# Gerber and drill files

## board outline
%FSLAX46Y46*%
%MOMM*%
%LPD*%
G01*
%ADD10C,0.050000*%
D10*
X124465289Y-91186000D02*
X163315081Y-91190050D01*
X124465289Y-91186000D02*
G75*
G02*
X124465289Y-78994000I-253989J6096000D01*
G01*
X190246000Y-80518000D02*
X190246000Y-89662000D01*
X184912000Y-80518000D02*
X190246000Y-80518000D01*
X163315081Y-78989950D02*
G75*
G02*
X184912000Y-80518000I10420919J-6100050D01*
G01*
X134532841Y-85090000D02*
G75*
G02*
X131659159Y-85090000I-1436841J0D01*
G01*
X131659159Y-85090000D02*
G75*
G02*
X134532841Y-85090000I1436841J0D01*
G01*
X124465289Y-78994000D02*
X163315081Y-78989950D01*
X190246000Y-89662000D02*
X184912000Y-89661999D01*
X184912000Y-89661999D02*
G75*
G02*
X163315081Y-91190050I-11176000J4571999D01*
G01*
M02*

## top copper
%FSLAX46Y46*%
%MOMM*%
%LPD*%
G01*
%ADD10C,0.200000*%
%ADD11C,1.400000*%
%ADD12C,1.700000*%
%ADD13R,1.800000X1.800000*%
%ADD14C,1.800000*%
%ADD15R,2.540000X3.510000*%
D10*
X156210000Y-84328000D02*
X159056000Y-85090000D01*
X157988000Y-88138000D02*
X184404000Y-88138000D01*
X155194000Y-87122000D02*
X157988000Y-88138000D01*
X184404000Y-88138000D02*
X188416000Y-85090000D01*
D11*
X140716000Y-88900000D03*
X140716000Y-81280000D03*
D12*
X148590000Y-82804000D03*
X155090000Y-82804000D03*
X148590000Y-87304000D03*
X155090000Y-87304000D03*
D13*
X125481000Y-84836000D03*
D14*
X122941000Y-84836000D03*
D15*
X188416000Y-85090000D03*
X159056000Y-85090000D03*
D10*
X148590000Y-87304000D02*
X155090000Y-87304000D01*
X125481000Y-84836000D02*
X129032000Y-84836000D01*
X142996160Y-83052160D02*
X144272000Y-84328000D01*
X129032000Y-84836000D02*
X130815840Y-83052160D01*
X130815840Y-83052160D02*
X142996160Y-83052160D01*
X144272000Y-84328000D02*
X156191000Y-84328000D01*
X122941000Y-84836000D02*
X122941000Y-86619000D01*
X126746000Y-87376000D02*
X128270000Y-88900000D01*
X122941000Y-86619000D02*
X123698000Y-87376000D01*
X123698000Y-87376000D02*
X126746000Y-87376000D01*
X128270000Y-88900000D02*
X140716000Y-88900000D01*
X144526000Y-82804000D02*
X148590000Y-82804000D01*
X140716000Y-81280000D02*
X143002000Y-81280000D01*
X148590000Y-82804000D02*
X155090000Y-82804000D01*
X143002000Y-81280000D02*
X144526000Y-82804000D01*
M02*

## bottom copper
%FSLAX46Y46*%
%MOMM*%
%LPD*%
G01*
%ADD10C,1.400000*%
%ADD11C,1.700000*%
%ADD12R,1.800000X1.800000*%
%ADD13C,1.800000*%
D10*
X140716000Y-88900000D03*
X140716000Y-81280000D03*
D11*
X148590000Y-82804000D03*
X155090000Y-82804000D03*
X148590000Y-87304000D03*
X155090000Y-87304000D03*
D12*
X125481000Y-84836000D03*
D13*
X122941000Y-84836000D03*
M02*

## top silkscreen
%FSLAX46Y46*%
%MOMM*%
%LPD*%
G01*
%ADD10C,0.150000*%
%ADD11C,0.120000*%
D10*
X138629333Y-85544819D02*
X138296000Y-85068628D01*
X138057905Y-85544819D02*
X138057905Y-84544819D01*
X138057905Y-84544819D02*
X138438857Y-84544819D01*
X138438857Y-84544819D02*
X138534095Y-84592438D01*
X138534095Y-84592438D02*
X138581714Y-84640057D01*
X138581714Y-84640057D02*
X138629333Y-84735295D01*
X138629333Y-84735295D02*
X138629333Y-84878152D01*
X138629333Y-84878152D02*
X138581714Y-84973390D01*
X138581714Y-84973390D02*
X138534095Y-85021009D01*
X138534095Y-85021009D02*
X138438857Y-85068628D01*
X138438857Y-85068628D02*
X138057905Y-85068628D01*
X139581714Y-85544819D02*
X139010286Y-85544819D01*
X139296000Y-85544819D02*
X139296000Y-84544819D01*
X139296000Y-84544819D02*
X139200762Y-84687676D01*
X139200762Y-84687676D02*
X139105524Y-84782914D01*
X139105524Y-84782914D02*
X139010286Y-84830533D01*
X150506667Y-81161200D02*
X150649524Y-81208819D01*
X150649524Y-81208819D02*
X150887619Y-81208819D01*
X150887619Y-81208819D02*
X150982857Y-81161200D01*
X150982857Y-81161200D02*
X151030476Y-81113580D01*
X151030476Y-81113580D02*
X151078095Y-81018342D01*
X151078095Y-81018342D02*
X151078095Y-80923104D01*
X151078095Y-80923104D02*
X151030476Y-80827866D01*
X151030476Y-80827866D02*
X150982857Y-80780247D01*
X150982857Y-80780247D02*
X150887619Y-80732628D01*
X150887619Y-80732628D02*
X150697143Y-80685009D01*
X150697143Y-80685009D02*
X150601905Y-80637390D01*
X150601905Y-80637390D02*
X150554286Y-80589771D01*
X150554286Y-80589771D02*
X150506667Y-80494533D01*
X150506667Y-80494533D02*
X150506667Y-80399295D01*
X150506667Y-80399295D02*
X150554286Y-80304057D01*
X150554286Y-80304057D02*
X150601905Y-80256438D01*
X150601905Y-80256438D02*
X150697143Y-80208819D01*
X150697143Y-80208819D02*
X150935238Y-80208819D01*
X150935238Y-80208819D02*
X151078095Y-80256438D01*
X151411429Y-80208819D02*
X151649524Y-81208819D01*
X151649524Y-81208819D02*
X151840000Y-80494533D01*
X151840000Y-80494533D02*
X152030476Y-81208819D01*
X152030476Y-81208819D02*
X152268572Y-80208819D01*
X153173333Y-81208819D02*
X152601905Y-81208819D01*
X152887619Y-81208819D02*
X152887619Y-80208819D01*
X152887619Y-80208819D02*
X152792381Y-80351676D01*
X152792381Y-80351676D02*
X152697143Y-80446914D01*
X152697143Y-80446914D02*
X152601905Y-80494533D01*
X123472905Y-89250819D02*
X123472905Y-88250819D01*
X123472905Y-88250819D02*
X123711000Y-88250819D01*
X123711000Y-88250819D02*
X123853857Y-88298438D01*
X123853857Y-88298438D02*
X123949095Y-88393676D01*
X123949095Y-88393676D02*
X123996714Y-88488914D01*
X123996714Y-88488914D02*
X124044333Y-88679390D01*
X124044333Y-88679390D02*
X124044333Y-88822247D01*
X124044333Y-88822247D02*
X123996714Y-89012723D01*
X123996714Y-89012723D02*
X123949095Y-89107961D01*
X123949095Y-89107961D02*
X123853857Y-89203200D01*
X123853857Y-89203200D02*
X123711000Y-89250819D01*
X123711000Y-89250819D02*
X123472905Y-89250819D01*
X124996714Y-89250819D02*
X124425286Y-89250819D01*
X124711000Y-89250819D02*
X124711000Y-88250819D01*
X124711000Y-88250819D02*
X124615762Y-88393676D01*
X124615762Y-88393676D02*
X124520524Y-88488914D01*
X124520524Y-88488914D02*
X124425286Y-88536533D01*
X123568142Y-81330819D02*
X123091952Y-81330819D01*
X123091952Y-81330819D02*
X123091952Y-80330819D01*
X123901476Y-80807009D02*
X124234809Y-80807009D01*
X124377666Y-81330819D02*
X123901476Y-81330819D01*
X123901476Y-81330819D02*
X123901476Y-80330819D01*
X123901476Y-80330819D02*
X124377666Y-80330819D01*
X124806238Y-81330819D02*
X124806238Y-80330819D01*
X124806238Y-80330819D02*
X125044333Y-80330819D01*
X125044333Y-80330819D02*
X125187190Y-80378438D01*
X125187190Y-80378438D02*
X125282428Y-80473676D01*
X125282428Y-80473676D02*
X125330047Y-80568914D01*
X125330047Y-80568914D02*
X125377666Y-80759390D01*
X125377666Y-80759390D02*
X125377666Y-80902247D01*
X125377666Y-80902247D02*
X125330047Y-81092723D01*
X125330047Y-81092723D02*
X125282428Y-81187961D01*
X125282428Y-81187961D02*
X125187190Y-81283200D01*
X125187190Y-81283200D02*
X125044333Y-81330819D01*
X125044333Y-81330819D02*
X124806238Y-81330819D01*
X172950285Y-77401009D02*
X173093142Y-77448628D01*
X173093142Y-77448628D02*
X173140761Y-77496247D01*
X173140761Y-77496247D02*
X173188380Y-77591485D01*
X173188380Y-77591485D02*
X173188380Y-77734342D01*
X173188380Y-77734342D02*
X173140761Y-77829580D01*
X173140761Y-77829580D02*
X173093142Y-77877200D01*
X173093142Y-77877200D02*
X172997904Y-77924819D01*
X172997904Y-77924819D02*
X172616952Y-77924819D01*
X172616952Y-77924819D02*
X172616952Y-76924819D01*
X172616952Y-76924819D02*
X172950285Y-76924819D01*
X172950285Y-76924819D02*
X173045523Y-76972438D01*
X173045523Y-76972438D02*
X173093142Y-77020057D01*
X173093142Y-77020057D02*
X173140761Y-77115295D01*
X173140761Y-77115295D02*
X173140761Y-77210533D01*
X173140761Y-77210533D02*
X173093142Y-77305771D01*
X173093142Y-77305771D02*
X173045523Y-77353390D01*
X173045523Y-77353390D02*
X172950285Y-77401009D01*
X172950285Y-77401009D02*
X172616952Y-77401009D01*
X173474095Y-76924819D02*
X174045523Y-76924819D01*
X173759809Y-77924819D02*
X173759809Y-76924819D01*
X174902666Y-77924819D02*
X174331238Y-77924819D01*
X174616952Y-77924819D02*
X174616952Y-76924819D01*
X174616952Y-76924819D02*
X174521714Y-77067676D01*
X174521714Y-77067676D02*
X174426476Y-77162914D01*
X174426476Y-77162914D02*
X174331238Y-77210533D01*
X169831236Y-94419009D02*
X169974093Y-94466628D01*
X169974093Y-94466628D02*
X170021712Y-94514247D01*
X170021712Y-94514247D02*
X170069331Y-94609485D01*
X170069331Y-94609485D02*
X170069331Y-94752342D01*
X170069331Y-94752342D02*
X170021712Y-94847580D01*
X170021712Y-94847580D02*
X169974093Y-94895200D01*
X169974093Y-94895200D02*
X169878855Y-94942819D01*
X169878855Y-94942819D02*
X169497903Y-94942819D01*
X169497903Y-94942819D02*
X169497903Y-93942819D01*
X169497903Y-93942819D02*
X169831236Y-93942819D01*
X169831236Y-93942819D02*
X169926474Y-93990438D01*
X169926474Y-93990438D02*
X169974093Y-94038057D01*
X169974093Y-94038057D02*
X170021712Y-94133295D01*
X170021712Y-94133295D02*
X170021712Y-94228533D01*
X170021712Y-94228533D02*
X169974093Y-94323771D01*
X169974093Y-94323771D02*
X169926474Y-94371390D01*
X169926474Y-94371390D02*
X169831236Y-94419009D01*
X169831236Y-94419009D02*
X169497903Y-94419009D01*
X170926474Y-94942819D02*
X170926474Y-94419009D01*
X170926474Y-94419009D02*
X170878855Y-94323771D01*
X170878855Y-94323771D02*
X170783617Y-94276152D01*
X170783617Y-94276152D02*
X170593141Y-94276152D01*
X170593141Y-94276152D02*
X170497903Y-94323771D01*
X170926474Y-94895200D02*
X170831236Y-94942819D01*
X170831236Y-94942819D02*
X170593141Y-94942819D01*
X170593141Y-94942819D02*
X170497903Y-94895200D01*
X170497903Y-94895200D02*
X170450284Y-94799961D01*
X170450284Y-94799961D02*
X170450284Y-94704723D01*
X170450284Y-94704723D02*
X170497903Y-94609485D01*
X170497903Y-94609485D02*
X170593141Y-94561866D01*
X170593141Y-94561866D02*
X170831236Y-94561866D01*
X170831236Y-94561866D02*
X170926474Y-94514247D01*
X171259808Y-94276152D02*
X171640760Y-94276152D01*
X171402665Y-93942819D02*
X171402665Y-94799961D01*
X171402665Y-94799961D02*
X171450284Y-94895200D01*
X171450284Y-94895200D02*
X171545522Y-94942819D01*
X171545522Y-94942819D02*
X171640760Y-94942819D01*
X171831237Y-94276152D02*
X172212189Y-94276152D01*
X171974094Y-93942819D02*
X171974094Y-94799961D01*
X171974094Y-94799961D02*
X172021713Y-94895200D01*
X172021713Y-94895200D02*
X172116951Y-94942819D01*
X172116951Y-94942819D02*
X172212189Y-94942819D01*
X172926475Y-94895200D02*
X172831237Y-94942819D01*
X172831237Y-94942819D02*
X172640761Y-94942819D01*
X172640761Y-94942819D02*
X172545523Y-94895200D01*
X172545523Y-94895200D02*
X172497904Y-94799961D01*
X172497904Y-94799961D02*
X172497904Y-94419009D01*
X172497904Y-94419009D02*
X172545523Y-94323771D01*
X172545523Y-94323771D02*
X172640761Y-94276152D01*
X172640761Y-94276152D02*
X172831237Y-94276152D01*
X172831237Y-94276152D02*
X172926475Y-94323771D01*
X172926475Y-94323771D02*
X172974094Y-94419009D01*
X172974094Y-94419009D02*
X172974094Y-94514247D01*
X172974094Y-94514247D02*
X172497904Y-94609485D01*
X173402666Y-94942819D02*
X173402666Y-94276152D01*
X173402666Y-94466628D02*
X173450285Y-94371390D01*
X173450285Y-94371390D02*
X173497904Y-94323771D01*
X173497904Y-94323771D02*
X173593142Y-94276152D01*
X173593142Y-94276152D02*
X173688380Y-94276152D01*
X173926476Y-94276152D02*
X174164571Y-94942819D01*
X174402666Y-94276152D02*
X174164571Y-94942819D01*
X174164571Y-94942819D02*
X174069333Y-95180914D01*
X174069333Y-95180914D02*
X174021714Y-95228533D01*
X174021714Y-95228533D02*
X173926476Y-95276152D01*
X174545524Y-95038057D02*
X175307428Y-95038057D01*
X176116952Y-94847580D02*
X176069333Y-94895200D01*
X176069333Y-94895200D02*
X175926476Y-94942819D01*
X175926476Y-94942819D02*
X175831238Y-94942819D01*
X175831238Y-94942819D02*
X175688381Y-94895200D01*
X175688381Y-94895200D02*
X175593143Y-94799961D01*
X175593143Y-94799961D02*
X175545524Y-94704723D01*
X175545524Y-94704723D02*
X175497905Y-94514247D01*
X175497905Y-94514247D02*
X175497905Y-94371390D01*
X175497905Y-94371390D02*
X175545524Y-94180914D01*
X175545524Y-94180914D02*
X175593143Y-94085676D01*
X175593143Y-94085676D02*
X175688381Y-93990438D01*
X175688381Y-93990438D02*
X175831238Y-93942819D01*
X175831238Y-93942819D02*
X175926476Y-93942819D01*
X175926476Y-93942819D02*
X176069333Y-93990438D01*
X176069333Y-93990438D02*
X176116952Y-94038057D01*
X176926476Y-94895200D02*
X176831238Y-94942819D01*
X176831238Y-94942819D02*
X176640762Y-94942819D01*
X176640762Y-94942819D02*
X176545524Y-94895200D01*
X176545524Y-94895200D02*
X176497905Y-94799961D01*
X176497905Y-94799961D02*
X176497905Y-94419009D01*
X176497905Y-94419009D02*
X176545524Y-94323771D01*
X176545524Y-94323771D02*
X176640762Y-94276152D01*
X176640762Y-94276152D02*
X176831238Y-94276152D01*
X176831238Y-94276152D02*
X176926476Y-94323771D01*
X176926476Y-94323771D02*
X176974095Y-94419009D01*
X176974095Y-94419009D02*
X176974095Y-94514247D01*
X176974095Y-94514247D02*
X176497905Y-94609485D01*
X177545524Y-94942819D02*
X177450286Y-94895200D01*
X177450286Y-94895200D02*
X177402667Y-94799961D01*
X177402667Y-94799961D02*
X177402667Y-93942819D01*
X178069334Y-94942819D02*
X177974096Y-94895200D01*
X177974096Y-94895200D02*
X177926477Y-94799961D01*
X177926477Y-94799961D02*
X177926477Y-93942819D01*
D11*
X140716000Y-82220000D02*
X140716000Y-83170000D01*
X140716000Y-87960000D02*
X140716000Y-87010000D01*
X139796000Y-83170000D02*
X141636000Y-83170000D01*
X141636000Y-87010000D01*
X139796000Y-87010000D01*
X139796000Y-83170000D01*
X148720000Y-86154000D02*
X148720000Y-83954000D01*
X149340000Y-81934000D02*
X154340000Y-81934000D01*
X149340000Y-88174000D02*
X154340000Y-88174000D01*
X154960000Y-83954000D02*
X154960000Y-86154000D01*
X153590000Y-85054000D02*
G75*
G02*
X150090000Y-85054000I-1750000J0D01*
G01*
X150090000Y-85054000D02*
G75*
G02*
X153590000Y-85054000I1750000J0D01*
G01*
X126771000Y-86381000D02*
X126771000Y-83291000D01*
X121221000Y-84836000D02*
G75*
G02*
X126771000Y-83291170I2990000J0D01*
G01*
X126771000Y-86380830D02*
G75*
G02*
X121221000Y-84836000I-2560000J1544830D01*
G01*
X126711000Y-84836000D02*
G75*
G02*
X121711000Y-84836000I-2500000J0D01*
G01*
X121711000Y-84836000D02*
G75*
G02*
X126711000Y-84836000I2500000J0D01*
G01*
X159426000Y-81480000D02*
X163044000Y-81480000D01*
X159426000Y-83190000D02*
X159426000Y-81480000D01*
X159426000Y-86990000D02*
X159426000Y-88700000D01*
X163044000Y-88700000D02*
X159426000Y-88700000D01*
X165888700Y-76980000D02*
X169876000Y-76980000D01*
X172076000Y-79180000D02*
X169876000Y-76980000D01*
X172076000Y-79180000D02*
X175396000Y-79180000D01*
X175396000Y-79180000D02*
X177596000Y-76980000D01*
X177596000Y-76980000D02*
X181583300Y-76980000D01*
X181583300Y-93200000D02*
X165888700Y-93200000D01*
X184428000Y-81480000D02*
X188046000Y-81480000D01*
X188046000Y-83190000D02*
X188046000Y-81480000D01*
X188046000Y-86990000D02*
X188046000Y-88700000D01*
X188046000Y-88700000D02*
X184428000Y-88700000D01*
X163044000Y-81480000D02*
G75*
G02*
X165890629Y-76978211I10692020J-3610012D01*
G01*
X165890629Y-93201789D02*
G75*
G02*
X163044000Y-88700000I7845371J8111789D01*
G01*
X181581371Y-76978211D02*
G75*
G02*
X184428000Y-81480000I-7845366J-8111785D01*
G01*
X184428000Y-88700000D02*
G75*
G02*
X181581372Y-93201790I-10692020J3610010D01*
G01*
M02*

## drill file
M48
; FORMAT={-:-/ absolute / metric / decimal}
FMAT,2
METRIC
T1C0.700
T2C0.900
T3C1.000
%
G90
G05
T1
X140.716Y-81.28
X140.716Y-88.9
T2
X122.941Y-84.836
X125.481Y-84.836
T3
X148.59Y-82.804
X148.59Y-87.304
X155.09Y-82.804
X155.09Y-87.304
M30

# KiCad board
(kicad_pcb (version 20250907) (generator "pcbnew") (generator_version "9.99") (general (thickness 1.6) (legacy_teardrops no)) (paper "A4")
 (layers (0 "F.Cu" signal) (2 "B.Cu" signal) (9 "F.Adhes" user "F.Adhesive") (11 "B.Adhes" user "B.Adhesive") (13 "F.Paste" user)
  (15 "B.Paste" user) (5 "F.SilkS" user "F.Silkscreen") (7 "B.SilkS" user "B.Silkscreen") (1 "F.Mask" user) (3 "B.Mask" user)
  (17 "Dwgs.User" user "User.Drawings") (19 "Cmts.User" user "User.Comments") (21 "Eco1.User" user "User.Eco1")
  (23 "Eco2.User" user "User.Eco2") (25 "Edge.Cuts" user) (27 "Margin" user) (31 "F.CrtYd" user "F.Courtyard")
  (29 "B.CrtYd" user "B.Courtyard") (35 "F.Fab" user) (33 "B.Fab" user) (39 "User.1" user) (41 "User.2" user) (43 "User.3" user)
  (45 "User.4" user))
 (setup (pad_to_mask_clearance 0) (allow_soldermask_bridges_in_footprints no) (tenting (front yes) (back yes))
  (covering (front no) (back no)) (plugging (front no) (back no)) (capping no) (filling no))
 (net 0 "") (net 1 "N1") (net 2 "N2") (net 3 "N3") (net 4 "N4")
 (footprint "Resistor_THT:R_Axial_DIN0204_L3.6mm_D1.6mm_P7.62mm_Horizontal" (layer "F.Cu") (at 140.716 88.9 90)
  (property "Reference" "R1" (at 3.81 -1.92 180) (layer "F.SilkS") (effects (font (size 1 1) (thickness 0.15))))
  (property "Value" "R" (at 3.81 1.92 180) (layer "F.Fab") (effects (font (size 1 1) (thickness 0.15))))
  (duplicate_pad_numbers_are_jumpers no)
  (fp_line (start 6.68 0) (end 5.73 0) (stroke (width 0.12) (type solid)) (layer "F.SilkS"))
  (fp_line (start 0.94 0) (end 1.89 0) (stroke (width 0.12) (type solid)) (layer "F.SilkS"))
  (fp_rect (start 1.89 -0.92) (end 5.73 0.92) (stroke (width 0.12) (type solid)) (fill no) (layer "F.SilkS"))
  (pad "1" thru_hole circle (at 0 0 90) (size 1.4 1.4) (drill 0.7) (layers "*.Cu" "*.Mask") (remove_unused_layers no) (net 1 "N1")
   (tenting (front none) (back none)))
  (pad "2" thru_hole circle (at 7.62 0 90) (size 1.4 1.4) (drill 0.7) (layers "*.Cu" "*.Mask") (remove_unused_layers no) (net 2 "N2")
   (tenting (front none) (back none))))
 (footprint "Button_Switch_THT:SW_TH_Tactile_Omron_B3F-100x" (layer "F.Cu") (at 148.59 82.804)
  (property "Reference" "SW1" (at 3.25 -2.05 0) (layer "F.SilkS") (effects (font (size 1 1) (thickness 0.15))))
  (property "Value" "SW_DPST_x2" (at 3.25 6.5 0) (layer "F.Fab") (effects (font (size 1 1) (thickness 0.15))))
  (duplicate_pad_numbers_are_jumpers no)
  (fp_line (start 0.13 3.35) (end 0.13 1.15) (stroke (width 0.12) (type solid)) (layer "F.SilkS"))
  (fp_line (start 0.75 -0.87) (end 5.75 -0.87) (stroke (width 0.12) (type solid)) (layer "F.SilkS"))
  (fp_line (start 0.75 5.37) (end 5.75 5.37) (stroke (width 0.12) (type solid)) (layer "F.SilkS"))
  (fp_line (start 6.37 1.15) (end 6.37 3.35) (stroke (width 0.12) (type solid)) (layer "F.SilkS"))
  (fp_circle (center 3.25 2.25) (end 5 2.25) (stroke (width 0.12) (type solid)) (fill no) (layer "F.SilkS"))
  (pad "1" thru_hole circle (at 0 0) (size 1.7 1.7) (drill 1) (layers "*.Cu" "*.Mask") (remove_unused_layers no) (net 2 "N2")
   (thermal_bridge_angle 90) (tenting (front none) (back none)))
  (pad "1" thru_hole circle (at 6.5 0) (size 1.7 1.7) (drill 1) (layers "*.Cu" "*.Mask") (remove_unused_layers no) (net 2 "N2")
   (tenting (front none) (back none)))
  (pad "2" thru_hole circle (at 0 4.5) (size 1.7 1.7) (drill 1) (layers "*.Cu" "*.Mask") (remove_unused_layers no) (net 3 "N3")
   (tenting (front none) (back none)))
  (pad "2" thru_hole circle (at 6.5 4.5) (size 1.7 1.7) (drill 1) (layers "*.Cu" "*.Mask") (remove_unused_layers no) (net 3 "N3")
   (tenting (front none) (back none))))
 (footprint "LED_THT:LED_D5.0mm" (layer "F.Cu") (at 125.481 84.836 180)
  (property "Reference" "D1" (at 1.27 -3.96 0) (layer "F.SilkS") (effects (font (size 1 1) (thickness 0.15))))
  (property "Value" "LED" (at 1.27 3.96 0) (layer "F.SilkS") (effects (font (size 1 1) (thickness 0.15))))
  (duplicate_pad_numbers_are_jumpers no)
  (fp_line (start -1.29 -1.545) (end -1.29 1.545) (stroke (width 0.12) (type solid)) (layer "F.SilkS"))
  (fp_arc (start 4.26 0) (mid 2.071779 2.880495) (end -1.29 1.54483) (stroke (width 0.12) (type solid)) (layer "F.SilkS"))
  (fp_arc (start -1.29 -1.54483) (mid 2.071779 -2.880495) (end 4.26 0) (stroke (width 0.12) (type solid)) (layer "F.SilkS"))
  (fp_circle (center 1.27 0) (end 3.77 0) (stroke (width 0.12) (type solid)) (fill no) (layer "F.SilkS"))
  (pad "1" thru_hole rect (at 0 0 180) (size 1.8 1.8) (drill 0.9) (layers "*.Cu" "*.Mask") (remove_unused_layers no) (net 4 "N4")
   (tenting (front none) (back none)))
  (pad "2" thru_hole circle (at 2.54 0 180) (size 1.8 1.8) (drill 0.9) (layers "*.Cu" "*.Mask") (remove_unused_layers no) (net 1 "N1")
   (tenting (front none) (back none))))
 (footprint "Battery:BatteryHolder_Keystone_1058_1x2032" (layer "F.Cu") (at 173.736 85.09 180)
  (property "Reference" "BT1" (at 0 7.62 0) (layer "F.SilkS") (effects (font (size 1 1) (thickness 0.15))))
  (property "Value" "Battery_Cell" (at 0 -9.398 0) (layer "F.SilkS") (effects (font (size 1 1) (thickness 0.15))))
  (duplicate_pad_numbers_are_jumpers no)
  (fp_line (start 14.31 3.61) (end 10.692 3.61) (stroke (width 0.12) (type solid)) (layer "F.SilkS"))
  (fp_line (start 14.31 1.9) (end 14.31 3.61) (stroke (width 0.12) (type solid)) (layer "F.SilkS"))
  (fp_line (start 14.31 -1.9) (end 14.31 -3.61) (stroke (width 0.12) (type solid)) (layer "F.SilkS"))
  (fp_line (start 10.692 -3.61) (end 14.31 -3.61) (stroke (width 0.12) (type solid)) (layer "F.SilkS"))
  (fp_line (start 7.8473 8.11) (end 3.86 8.11) (stroke (width 0.12) (type solid)) (layer "F.SilkS"))
  (fp_line (start 1.66 5.91) (end 3.86 8.11) (stroke (width 0.12) (type solid)) (layer "F.SilkS"))
  (fp_line (start 1.66 5.91) (end -1.66 5.91) (stroke (width 0.12) (type solid)) (layer "F.SilkS"))
  (fp_line (start -1.66 5.91) (end -3.86 8.11) (stroke (width 0.12) (type solid)) (layer "F.SilkS"))
  (fp_line (start -3.86 8.11) (end -7.8473 8.11) (stroke (width 0.12) (type solid)) (layer "F.SilkS"))
  (fp_line (start -7.8473 -8.11) (end 7.8473 -8.11) (stroke (width 0.12) (type solid)) (layer "F.SilkS"))
  (fp_line (start -10.692 3.61) (end -14.31 3.61) (stroke (width 0.12) (type solid)) (layer "F.SilkS"))
  (fp_line (start -14.31 1.9) (end -14.31 3.61) (stroke (width 0.12) (type solid)) (layer "F.SilkS"))
  (fp_line (start -14.31 -1.9) (end -14.31 -3.61) (stroke (width 0.12) (type solid)) (layer "F.SilkS"))
  (fp_line (start -14.31 -3.61) (end -10.692 -3.61) (stroke (width 0.12) (type solid)) (layer "F.SilkS"))
  (fp_arc (start 10.692 3.61) (mid 9.538084 6.031244) (end 7.845371 8.111789) (stroke (width 0.12) (type solid)) (layer "F.SilkS"))
  (fp_arc (start 7.845371 -8.111789) (mid 9.538085 -6.031244) (end 10.692 -3.61) (stroke (width 0.12) (type solid)) (layer "F.SilkS"))
  (fp_arc (start -7.845371 8.111789) (mid -9.538085 6.031244) (end -10.692 3.61) (stroke (width 0.12) (type solid)) (layer "F.SilkS"))
  (fp_arc (start -10.692 -3.61) (mid -9.538084 -6.031244) (end -7.845371 -8.111789) (stroke (width 0.12) (type solid)) (layer "F.SilkS"))
  (pad "1" smd rect (at -14.68 0 180) (size 2.54 3.51) (layers "F.Cu" "F.Mask" "F.Paste") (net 3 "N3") (tenting (front none) (back none)))
  (pad "2" smd rect (at 14.68 0 180) (size 2.54 3.51) (layers "F.Cu" "F.Mask" "F.Paste") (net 4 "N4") (tenting (front none) (back none))))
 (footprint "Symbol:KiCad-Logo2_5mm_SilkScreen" (layer "B.Cu") (at 174.244 84.836 180)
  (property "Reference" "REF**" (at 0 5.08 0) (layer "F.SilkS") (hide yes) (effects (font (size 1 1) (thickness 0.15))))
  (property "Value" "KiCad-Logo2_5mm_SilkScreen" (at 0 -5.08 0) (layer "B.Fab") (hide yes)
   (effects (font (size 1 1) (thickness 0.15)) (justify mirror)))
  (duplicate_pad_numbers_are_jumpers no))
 (gr_line (start 156.21 84.328) (end 159.056 85.09) (stroke (width 0.2) (type default)) (layer "F.Cu") (net 4))
 (gr_line (start 157.988 88.138) (end 184.404 88.138) (stroke (width 0.2) (type default)) (layer "F.Cu") (net 3))
 (gr_line (start 155.194 87.122) (end 157.988 88.138) (stroke (width 0.2) (type default)) (layer "F.Cu") (net 3))
 (gr_line (start 184.404 88.138) (end 188.416 85.09) (stroke (width 0.2) (type default)) (layer "F.Cu") (net 3))
 (gr_line (start 124.465289 91.186) (end 163.315081 91.19005) (stroke (width 0.05) (type default)) (layer "Edge.Cuts"))
 (gr_arc (start 124.465289 91.186) (mid 118.11 85.09) (end 124.465289 78.994) (stroke (width 0.05) (type default)) (layer "Edge.Cuts"))
 (gr_line (start 190.246 80.518) (end 190.246 89.662) (stroke (width 0.05) (type default)) (layer "Edge.Cuts"))
 (gr_line (start 184.912 80.518) (end 190.246 80.518) (stroke (width 0.05) (type default)) (layer "Edge.Cuts"))
 (gr_arc (start 163.315081 78.98995) (mid 174.588215 73.045089) (end 184.912 80.518) (stroke (width 0.05) (type default))
  (layer "Edge.Cuts"))
 (gr_circle (center 133.096 85.09) (end 134.112 86.106) (stroke (width 0.05) (type default)) (fill no) (layer "Edge.Cuts"))
 (gr_line (start 124.465289 78.994) (end 163.315081 78.98995) (stroke (width 0.05) (type default)) (layer "Edge.Cuts"))
 (gr_line (start 190.246 89.662) (end 184.912 89.661999) (stroke (width 0.05) (type default)) (layer "Edge.Cuts"))
 (gr_arc (start 184.912 89.661999) (mid 174.588216 97.134911) (end 163.315081 91.19005) (stroke (width 0.05) (type default))
  (layer "Edge.Cuts"))
 (segment (start 148.59 87.304) (end 155.09 87.304) (width 0.2) (layer "F.Cu") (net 3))
 (segment (start 125.481 84.836) (end 129.032 84.836) (width 0.2) (layer "F.Cu") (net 4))
 (segment (start 142.99616 83.05216) (end 144.272 84.328) (width 0.2) (layer "F.Cu") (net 4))
 (segment (start 129.032 84.836) (end 130.81584 83.05216) (width 0.2) (layer "F.Cu") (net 4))
 (segment (start 130.81584 83.05216) (end 142.99616 83.05216) (width 0.2) (layer "F.Cu") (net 4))
 (segment (start 144.272 84.328) (end 156.191 84.328) (width 0.2) (layer "F.Cu") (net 4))
 (segment (start 122.941 84.836) (end 122.941 86.619) (width 0.2) (layer "F.Cu") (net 1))
 (segment (start 126.746 87.376) (end 128.27 88.9) (width 0.2) (layer "F.Cu") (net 1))
 (segment (start 122.941 86.619) (end 123.698 87.376) (width 0.2) (layer "F.Cu") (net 1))
 (segment (start 123.698 87.376) (end 126.746 87.376) (width 0.2) (layer "F.Cu") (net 1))
 (segment (start 128.27 88.9) (end 140.716 88.9) (width 0.2) (layer "F.Cu") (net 1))
 (segment (start 144.526 82.804) (end 148.59 82.804) (width 0.2) (layer "F.Cu") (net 2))
 (segment (start 140.716 81.28) (end 143.002 81.28) (width 0.2) (layer "F.Cu") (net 2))
 (segment (start 148.59 82.804) (end 155.09 82.804) (width 0.2) (layer "F.Cu") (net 2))
 (segment (start 143.002 81.28) (end 144.526 82.804) (width 0.2) (layer "F.Cu") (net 2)))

